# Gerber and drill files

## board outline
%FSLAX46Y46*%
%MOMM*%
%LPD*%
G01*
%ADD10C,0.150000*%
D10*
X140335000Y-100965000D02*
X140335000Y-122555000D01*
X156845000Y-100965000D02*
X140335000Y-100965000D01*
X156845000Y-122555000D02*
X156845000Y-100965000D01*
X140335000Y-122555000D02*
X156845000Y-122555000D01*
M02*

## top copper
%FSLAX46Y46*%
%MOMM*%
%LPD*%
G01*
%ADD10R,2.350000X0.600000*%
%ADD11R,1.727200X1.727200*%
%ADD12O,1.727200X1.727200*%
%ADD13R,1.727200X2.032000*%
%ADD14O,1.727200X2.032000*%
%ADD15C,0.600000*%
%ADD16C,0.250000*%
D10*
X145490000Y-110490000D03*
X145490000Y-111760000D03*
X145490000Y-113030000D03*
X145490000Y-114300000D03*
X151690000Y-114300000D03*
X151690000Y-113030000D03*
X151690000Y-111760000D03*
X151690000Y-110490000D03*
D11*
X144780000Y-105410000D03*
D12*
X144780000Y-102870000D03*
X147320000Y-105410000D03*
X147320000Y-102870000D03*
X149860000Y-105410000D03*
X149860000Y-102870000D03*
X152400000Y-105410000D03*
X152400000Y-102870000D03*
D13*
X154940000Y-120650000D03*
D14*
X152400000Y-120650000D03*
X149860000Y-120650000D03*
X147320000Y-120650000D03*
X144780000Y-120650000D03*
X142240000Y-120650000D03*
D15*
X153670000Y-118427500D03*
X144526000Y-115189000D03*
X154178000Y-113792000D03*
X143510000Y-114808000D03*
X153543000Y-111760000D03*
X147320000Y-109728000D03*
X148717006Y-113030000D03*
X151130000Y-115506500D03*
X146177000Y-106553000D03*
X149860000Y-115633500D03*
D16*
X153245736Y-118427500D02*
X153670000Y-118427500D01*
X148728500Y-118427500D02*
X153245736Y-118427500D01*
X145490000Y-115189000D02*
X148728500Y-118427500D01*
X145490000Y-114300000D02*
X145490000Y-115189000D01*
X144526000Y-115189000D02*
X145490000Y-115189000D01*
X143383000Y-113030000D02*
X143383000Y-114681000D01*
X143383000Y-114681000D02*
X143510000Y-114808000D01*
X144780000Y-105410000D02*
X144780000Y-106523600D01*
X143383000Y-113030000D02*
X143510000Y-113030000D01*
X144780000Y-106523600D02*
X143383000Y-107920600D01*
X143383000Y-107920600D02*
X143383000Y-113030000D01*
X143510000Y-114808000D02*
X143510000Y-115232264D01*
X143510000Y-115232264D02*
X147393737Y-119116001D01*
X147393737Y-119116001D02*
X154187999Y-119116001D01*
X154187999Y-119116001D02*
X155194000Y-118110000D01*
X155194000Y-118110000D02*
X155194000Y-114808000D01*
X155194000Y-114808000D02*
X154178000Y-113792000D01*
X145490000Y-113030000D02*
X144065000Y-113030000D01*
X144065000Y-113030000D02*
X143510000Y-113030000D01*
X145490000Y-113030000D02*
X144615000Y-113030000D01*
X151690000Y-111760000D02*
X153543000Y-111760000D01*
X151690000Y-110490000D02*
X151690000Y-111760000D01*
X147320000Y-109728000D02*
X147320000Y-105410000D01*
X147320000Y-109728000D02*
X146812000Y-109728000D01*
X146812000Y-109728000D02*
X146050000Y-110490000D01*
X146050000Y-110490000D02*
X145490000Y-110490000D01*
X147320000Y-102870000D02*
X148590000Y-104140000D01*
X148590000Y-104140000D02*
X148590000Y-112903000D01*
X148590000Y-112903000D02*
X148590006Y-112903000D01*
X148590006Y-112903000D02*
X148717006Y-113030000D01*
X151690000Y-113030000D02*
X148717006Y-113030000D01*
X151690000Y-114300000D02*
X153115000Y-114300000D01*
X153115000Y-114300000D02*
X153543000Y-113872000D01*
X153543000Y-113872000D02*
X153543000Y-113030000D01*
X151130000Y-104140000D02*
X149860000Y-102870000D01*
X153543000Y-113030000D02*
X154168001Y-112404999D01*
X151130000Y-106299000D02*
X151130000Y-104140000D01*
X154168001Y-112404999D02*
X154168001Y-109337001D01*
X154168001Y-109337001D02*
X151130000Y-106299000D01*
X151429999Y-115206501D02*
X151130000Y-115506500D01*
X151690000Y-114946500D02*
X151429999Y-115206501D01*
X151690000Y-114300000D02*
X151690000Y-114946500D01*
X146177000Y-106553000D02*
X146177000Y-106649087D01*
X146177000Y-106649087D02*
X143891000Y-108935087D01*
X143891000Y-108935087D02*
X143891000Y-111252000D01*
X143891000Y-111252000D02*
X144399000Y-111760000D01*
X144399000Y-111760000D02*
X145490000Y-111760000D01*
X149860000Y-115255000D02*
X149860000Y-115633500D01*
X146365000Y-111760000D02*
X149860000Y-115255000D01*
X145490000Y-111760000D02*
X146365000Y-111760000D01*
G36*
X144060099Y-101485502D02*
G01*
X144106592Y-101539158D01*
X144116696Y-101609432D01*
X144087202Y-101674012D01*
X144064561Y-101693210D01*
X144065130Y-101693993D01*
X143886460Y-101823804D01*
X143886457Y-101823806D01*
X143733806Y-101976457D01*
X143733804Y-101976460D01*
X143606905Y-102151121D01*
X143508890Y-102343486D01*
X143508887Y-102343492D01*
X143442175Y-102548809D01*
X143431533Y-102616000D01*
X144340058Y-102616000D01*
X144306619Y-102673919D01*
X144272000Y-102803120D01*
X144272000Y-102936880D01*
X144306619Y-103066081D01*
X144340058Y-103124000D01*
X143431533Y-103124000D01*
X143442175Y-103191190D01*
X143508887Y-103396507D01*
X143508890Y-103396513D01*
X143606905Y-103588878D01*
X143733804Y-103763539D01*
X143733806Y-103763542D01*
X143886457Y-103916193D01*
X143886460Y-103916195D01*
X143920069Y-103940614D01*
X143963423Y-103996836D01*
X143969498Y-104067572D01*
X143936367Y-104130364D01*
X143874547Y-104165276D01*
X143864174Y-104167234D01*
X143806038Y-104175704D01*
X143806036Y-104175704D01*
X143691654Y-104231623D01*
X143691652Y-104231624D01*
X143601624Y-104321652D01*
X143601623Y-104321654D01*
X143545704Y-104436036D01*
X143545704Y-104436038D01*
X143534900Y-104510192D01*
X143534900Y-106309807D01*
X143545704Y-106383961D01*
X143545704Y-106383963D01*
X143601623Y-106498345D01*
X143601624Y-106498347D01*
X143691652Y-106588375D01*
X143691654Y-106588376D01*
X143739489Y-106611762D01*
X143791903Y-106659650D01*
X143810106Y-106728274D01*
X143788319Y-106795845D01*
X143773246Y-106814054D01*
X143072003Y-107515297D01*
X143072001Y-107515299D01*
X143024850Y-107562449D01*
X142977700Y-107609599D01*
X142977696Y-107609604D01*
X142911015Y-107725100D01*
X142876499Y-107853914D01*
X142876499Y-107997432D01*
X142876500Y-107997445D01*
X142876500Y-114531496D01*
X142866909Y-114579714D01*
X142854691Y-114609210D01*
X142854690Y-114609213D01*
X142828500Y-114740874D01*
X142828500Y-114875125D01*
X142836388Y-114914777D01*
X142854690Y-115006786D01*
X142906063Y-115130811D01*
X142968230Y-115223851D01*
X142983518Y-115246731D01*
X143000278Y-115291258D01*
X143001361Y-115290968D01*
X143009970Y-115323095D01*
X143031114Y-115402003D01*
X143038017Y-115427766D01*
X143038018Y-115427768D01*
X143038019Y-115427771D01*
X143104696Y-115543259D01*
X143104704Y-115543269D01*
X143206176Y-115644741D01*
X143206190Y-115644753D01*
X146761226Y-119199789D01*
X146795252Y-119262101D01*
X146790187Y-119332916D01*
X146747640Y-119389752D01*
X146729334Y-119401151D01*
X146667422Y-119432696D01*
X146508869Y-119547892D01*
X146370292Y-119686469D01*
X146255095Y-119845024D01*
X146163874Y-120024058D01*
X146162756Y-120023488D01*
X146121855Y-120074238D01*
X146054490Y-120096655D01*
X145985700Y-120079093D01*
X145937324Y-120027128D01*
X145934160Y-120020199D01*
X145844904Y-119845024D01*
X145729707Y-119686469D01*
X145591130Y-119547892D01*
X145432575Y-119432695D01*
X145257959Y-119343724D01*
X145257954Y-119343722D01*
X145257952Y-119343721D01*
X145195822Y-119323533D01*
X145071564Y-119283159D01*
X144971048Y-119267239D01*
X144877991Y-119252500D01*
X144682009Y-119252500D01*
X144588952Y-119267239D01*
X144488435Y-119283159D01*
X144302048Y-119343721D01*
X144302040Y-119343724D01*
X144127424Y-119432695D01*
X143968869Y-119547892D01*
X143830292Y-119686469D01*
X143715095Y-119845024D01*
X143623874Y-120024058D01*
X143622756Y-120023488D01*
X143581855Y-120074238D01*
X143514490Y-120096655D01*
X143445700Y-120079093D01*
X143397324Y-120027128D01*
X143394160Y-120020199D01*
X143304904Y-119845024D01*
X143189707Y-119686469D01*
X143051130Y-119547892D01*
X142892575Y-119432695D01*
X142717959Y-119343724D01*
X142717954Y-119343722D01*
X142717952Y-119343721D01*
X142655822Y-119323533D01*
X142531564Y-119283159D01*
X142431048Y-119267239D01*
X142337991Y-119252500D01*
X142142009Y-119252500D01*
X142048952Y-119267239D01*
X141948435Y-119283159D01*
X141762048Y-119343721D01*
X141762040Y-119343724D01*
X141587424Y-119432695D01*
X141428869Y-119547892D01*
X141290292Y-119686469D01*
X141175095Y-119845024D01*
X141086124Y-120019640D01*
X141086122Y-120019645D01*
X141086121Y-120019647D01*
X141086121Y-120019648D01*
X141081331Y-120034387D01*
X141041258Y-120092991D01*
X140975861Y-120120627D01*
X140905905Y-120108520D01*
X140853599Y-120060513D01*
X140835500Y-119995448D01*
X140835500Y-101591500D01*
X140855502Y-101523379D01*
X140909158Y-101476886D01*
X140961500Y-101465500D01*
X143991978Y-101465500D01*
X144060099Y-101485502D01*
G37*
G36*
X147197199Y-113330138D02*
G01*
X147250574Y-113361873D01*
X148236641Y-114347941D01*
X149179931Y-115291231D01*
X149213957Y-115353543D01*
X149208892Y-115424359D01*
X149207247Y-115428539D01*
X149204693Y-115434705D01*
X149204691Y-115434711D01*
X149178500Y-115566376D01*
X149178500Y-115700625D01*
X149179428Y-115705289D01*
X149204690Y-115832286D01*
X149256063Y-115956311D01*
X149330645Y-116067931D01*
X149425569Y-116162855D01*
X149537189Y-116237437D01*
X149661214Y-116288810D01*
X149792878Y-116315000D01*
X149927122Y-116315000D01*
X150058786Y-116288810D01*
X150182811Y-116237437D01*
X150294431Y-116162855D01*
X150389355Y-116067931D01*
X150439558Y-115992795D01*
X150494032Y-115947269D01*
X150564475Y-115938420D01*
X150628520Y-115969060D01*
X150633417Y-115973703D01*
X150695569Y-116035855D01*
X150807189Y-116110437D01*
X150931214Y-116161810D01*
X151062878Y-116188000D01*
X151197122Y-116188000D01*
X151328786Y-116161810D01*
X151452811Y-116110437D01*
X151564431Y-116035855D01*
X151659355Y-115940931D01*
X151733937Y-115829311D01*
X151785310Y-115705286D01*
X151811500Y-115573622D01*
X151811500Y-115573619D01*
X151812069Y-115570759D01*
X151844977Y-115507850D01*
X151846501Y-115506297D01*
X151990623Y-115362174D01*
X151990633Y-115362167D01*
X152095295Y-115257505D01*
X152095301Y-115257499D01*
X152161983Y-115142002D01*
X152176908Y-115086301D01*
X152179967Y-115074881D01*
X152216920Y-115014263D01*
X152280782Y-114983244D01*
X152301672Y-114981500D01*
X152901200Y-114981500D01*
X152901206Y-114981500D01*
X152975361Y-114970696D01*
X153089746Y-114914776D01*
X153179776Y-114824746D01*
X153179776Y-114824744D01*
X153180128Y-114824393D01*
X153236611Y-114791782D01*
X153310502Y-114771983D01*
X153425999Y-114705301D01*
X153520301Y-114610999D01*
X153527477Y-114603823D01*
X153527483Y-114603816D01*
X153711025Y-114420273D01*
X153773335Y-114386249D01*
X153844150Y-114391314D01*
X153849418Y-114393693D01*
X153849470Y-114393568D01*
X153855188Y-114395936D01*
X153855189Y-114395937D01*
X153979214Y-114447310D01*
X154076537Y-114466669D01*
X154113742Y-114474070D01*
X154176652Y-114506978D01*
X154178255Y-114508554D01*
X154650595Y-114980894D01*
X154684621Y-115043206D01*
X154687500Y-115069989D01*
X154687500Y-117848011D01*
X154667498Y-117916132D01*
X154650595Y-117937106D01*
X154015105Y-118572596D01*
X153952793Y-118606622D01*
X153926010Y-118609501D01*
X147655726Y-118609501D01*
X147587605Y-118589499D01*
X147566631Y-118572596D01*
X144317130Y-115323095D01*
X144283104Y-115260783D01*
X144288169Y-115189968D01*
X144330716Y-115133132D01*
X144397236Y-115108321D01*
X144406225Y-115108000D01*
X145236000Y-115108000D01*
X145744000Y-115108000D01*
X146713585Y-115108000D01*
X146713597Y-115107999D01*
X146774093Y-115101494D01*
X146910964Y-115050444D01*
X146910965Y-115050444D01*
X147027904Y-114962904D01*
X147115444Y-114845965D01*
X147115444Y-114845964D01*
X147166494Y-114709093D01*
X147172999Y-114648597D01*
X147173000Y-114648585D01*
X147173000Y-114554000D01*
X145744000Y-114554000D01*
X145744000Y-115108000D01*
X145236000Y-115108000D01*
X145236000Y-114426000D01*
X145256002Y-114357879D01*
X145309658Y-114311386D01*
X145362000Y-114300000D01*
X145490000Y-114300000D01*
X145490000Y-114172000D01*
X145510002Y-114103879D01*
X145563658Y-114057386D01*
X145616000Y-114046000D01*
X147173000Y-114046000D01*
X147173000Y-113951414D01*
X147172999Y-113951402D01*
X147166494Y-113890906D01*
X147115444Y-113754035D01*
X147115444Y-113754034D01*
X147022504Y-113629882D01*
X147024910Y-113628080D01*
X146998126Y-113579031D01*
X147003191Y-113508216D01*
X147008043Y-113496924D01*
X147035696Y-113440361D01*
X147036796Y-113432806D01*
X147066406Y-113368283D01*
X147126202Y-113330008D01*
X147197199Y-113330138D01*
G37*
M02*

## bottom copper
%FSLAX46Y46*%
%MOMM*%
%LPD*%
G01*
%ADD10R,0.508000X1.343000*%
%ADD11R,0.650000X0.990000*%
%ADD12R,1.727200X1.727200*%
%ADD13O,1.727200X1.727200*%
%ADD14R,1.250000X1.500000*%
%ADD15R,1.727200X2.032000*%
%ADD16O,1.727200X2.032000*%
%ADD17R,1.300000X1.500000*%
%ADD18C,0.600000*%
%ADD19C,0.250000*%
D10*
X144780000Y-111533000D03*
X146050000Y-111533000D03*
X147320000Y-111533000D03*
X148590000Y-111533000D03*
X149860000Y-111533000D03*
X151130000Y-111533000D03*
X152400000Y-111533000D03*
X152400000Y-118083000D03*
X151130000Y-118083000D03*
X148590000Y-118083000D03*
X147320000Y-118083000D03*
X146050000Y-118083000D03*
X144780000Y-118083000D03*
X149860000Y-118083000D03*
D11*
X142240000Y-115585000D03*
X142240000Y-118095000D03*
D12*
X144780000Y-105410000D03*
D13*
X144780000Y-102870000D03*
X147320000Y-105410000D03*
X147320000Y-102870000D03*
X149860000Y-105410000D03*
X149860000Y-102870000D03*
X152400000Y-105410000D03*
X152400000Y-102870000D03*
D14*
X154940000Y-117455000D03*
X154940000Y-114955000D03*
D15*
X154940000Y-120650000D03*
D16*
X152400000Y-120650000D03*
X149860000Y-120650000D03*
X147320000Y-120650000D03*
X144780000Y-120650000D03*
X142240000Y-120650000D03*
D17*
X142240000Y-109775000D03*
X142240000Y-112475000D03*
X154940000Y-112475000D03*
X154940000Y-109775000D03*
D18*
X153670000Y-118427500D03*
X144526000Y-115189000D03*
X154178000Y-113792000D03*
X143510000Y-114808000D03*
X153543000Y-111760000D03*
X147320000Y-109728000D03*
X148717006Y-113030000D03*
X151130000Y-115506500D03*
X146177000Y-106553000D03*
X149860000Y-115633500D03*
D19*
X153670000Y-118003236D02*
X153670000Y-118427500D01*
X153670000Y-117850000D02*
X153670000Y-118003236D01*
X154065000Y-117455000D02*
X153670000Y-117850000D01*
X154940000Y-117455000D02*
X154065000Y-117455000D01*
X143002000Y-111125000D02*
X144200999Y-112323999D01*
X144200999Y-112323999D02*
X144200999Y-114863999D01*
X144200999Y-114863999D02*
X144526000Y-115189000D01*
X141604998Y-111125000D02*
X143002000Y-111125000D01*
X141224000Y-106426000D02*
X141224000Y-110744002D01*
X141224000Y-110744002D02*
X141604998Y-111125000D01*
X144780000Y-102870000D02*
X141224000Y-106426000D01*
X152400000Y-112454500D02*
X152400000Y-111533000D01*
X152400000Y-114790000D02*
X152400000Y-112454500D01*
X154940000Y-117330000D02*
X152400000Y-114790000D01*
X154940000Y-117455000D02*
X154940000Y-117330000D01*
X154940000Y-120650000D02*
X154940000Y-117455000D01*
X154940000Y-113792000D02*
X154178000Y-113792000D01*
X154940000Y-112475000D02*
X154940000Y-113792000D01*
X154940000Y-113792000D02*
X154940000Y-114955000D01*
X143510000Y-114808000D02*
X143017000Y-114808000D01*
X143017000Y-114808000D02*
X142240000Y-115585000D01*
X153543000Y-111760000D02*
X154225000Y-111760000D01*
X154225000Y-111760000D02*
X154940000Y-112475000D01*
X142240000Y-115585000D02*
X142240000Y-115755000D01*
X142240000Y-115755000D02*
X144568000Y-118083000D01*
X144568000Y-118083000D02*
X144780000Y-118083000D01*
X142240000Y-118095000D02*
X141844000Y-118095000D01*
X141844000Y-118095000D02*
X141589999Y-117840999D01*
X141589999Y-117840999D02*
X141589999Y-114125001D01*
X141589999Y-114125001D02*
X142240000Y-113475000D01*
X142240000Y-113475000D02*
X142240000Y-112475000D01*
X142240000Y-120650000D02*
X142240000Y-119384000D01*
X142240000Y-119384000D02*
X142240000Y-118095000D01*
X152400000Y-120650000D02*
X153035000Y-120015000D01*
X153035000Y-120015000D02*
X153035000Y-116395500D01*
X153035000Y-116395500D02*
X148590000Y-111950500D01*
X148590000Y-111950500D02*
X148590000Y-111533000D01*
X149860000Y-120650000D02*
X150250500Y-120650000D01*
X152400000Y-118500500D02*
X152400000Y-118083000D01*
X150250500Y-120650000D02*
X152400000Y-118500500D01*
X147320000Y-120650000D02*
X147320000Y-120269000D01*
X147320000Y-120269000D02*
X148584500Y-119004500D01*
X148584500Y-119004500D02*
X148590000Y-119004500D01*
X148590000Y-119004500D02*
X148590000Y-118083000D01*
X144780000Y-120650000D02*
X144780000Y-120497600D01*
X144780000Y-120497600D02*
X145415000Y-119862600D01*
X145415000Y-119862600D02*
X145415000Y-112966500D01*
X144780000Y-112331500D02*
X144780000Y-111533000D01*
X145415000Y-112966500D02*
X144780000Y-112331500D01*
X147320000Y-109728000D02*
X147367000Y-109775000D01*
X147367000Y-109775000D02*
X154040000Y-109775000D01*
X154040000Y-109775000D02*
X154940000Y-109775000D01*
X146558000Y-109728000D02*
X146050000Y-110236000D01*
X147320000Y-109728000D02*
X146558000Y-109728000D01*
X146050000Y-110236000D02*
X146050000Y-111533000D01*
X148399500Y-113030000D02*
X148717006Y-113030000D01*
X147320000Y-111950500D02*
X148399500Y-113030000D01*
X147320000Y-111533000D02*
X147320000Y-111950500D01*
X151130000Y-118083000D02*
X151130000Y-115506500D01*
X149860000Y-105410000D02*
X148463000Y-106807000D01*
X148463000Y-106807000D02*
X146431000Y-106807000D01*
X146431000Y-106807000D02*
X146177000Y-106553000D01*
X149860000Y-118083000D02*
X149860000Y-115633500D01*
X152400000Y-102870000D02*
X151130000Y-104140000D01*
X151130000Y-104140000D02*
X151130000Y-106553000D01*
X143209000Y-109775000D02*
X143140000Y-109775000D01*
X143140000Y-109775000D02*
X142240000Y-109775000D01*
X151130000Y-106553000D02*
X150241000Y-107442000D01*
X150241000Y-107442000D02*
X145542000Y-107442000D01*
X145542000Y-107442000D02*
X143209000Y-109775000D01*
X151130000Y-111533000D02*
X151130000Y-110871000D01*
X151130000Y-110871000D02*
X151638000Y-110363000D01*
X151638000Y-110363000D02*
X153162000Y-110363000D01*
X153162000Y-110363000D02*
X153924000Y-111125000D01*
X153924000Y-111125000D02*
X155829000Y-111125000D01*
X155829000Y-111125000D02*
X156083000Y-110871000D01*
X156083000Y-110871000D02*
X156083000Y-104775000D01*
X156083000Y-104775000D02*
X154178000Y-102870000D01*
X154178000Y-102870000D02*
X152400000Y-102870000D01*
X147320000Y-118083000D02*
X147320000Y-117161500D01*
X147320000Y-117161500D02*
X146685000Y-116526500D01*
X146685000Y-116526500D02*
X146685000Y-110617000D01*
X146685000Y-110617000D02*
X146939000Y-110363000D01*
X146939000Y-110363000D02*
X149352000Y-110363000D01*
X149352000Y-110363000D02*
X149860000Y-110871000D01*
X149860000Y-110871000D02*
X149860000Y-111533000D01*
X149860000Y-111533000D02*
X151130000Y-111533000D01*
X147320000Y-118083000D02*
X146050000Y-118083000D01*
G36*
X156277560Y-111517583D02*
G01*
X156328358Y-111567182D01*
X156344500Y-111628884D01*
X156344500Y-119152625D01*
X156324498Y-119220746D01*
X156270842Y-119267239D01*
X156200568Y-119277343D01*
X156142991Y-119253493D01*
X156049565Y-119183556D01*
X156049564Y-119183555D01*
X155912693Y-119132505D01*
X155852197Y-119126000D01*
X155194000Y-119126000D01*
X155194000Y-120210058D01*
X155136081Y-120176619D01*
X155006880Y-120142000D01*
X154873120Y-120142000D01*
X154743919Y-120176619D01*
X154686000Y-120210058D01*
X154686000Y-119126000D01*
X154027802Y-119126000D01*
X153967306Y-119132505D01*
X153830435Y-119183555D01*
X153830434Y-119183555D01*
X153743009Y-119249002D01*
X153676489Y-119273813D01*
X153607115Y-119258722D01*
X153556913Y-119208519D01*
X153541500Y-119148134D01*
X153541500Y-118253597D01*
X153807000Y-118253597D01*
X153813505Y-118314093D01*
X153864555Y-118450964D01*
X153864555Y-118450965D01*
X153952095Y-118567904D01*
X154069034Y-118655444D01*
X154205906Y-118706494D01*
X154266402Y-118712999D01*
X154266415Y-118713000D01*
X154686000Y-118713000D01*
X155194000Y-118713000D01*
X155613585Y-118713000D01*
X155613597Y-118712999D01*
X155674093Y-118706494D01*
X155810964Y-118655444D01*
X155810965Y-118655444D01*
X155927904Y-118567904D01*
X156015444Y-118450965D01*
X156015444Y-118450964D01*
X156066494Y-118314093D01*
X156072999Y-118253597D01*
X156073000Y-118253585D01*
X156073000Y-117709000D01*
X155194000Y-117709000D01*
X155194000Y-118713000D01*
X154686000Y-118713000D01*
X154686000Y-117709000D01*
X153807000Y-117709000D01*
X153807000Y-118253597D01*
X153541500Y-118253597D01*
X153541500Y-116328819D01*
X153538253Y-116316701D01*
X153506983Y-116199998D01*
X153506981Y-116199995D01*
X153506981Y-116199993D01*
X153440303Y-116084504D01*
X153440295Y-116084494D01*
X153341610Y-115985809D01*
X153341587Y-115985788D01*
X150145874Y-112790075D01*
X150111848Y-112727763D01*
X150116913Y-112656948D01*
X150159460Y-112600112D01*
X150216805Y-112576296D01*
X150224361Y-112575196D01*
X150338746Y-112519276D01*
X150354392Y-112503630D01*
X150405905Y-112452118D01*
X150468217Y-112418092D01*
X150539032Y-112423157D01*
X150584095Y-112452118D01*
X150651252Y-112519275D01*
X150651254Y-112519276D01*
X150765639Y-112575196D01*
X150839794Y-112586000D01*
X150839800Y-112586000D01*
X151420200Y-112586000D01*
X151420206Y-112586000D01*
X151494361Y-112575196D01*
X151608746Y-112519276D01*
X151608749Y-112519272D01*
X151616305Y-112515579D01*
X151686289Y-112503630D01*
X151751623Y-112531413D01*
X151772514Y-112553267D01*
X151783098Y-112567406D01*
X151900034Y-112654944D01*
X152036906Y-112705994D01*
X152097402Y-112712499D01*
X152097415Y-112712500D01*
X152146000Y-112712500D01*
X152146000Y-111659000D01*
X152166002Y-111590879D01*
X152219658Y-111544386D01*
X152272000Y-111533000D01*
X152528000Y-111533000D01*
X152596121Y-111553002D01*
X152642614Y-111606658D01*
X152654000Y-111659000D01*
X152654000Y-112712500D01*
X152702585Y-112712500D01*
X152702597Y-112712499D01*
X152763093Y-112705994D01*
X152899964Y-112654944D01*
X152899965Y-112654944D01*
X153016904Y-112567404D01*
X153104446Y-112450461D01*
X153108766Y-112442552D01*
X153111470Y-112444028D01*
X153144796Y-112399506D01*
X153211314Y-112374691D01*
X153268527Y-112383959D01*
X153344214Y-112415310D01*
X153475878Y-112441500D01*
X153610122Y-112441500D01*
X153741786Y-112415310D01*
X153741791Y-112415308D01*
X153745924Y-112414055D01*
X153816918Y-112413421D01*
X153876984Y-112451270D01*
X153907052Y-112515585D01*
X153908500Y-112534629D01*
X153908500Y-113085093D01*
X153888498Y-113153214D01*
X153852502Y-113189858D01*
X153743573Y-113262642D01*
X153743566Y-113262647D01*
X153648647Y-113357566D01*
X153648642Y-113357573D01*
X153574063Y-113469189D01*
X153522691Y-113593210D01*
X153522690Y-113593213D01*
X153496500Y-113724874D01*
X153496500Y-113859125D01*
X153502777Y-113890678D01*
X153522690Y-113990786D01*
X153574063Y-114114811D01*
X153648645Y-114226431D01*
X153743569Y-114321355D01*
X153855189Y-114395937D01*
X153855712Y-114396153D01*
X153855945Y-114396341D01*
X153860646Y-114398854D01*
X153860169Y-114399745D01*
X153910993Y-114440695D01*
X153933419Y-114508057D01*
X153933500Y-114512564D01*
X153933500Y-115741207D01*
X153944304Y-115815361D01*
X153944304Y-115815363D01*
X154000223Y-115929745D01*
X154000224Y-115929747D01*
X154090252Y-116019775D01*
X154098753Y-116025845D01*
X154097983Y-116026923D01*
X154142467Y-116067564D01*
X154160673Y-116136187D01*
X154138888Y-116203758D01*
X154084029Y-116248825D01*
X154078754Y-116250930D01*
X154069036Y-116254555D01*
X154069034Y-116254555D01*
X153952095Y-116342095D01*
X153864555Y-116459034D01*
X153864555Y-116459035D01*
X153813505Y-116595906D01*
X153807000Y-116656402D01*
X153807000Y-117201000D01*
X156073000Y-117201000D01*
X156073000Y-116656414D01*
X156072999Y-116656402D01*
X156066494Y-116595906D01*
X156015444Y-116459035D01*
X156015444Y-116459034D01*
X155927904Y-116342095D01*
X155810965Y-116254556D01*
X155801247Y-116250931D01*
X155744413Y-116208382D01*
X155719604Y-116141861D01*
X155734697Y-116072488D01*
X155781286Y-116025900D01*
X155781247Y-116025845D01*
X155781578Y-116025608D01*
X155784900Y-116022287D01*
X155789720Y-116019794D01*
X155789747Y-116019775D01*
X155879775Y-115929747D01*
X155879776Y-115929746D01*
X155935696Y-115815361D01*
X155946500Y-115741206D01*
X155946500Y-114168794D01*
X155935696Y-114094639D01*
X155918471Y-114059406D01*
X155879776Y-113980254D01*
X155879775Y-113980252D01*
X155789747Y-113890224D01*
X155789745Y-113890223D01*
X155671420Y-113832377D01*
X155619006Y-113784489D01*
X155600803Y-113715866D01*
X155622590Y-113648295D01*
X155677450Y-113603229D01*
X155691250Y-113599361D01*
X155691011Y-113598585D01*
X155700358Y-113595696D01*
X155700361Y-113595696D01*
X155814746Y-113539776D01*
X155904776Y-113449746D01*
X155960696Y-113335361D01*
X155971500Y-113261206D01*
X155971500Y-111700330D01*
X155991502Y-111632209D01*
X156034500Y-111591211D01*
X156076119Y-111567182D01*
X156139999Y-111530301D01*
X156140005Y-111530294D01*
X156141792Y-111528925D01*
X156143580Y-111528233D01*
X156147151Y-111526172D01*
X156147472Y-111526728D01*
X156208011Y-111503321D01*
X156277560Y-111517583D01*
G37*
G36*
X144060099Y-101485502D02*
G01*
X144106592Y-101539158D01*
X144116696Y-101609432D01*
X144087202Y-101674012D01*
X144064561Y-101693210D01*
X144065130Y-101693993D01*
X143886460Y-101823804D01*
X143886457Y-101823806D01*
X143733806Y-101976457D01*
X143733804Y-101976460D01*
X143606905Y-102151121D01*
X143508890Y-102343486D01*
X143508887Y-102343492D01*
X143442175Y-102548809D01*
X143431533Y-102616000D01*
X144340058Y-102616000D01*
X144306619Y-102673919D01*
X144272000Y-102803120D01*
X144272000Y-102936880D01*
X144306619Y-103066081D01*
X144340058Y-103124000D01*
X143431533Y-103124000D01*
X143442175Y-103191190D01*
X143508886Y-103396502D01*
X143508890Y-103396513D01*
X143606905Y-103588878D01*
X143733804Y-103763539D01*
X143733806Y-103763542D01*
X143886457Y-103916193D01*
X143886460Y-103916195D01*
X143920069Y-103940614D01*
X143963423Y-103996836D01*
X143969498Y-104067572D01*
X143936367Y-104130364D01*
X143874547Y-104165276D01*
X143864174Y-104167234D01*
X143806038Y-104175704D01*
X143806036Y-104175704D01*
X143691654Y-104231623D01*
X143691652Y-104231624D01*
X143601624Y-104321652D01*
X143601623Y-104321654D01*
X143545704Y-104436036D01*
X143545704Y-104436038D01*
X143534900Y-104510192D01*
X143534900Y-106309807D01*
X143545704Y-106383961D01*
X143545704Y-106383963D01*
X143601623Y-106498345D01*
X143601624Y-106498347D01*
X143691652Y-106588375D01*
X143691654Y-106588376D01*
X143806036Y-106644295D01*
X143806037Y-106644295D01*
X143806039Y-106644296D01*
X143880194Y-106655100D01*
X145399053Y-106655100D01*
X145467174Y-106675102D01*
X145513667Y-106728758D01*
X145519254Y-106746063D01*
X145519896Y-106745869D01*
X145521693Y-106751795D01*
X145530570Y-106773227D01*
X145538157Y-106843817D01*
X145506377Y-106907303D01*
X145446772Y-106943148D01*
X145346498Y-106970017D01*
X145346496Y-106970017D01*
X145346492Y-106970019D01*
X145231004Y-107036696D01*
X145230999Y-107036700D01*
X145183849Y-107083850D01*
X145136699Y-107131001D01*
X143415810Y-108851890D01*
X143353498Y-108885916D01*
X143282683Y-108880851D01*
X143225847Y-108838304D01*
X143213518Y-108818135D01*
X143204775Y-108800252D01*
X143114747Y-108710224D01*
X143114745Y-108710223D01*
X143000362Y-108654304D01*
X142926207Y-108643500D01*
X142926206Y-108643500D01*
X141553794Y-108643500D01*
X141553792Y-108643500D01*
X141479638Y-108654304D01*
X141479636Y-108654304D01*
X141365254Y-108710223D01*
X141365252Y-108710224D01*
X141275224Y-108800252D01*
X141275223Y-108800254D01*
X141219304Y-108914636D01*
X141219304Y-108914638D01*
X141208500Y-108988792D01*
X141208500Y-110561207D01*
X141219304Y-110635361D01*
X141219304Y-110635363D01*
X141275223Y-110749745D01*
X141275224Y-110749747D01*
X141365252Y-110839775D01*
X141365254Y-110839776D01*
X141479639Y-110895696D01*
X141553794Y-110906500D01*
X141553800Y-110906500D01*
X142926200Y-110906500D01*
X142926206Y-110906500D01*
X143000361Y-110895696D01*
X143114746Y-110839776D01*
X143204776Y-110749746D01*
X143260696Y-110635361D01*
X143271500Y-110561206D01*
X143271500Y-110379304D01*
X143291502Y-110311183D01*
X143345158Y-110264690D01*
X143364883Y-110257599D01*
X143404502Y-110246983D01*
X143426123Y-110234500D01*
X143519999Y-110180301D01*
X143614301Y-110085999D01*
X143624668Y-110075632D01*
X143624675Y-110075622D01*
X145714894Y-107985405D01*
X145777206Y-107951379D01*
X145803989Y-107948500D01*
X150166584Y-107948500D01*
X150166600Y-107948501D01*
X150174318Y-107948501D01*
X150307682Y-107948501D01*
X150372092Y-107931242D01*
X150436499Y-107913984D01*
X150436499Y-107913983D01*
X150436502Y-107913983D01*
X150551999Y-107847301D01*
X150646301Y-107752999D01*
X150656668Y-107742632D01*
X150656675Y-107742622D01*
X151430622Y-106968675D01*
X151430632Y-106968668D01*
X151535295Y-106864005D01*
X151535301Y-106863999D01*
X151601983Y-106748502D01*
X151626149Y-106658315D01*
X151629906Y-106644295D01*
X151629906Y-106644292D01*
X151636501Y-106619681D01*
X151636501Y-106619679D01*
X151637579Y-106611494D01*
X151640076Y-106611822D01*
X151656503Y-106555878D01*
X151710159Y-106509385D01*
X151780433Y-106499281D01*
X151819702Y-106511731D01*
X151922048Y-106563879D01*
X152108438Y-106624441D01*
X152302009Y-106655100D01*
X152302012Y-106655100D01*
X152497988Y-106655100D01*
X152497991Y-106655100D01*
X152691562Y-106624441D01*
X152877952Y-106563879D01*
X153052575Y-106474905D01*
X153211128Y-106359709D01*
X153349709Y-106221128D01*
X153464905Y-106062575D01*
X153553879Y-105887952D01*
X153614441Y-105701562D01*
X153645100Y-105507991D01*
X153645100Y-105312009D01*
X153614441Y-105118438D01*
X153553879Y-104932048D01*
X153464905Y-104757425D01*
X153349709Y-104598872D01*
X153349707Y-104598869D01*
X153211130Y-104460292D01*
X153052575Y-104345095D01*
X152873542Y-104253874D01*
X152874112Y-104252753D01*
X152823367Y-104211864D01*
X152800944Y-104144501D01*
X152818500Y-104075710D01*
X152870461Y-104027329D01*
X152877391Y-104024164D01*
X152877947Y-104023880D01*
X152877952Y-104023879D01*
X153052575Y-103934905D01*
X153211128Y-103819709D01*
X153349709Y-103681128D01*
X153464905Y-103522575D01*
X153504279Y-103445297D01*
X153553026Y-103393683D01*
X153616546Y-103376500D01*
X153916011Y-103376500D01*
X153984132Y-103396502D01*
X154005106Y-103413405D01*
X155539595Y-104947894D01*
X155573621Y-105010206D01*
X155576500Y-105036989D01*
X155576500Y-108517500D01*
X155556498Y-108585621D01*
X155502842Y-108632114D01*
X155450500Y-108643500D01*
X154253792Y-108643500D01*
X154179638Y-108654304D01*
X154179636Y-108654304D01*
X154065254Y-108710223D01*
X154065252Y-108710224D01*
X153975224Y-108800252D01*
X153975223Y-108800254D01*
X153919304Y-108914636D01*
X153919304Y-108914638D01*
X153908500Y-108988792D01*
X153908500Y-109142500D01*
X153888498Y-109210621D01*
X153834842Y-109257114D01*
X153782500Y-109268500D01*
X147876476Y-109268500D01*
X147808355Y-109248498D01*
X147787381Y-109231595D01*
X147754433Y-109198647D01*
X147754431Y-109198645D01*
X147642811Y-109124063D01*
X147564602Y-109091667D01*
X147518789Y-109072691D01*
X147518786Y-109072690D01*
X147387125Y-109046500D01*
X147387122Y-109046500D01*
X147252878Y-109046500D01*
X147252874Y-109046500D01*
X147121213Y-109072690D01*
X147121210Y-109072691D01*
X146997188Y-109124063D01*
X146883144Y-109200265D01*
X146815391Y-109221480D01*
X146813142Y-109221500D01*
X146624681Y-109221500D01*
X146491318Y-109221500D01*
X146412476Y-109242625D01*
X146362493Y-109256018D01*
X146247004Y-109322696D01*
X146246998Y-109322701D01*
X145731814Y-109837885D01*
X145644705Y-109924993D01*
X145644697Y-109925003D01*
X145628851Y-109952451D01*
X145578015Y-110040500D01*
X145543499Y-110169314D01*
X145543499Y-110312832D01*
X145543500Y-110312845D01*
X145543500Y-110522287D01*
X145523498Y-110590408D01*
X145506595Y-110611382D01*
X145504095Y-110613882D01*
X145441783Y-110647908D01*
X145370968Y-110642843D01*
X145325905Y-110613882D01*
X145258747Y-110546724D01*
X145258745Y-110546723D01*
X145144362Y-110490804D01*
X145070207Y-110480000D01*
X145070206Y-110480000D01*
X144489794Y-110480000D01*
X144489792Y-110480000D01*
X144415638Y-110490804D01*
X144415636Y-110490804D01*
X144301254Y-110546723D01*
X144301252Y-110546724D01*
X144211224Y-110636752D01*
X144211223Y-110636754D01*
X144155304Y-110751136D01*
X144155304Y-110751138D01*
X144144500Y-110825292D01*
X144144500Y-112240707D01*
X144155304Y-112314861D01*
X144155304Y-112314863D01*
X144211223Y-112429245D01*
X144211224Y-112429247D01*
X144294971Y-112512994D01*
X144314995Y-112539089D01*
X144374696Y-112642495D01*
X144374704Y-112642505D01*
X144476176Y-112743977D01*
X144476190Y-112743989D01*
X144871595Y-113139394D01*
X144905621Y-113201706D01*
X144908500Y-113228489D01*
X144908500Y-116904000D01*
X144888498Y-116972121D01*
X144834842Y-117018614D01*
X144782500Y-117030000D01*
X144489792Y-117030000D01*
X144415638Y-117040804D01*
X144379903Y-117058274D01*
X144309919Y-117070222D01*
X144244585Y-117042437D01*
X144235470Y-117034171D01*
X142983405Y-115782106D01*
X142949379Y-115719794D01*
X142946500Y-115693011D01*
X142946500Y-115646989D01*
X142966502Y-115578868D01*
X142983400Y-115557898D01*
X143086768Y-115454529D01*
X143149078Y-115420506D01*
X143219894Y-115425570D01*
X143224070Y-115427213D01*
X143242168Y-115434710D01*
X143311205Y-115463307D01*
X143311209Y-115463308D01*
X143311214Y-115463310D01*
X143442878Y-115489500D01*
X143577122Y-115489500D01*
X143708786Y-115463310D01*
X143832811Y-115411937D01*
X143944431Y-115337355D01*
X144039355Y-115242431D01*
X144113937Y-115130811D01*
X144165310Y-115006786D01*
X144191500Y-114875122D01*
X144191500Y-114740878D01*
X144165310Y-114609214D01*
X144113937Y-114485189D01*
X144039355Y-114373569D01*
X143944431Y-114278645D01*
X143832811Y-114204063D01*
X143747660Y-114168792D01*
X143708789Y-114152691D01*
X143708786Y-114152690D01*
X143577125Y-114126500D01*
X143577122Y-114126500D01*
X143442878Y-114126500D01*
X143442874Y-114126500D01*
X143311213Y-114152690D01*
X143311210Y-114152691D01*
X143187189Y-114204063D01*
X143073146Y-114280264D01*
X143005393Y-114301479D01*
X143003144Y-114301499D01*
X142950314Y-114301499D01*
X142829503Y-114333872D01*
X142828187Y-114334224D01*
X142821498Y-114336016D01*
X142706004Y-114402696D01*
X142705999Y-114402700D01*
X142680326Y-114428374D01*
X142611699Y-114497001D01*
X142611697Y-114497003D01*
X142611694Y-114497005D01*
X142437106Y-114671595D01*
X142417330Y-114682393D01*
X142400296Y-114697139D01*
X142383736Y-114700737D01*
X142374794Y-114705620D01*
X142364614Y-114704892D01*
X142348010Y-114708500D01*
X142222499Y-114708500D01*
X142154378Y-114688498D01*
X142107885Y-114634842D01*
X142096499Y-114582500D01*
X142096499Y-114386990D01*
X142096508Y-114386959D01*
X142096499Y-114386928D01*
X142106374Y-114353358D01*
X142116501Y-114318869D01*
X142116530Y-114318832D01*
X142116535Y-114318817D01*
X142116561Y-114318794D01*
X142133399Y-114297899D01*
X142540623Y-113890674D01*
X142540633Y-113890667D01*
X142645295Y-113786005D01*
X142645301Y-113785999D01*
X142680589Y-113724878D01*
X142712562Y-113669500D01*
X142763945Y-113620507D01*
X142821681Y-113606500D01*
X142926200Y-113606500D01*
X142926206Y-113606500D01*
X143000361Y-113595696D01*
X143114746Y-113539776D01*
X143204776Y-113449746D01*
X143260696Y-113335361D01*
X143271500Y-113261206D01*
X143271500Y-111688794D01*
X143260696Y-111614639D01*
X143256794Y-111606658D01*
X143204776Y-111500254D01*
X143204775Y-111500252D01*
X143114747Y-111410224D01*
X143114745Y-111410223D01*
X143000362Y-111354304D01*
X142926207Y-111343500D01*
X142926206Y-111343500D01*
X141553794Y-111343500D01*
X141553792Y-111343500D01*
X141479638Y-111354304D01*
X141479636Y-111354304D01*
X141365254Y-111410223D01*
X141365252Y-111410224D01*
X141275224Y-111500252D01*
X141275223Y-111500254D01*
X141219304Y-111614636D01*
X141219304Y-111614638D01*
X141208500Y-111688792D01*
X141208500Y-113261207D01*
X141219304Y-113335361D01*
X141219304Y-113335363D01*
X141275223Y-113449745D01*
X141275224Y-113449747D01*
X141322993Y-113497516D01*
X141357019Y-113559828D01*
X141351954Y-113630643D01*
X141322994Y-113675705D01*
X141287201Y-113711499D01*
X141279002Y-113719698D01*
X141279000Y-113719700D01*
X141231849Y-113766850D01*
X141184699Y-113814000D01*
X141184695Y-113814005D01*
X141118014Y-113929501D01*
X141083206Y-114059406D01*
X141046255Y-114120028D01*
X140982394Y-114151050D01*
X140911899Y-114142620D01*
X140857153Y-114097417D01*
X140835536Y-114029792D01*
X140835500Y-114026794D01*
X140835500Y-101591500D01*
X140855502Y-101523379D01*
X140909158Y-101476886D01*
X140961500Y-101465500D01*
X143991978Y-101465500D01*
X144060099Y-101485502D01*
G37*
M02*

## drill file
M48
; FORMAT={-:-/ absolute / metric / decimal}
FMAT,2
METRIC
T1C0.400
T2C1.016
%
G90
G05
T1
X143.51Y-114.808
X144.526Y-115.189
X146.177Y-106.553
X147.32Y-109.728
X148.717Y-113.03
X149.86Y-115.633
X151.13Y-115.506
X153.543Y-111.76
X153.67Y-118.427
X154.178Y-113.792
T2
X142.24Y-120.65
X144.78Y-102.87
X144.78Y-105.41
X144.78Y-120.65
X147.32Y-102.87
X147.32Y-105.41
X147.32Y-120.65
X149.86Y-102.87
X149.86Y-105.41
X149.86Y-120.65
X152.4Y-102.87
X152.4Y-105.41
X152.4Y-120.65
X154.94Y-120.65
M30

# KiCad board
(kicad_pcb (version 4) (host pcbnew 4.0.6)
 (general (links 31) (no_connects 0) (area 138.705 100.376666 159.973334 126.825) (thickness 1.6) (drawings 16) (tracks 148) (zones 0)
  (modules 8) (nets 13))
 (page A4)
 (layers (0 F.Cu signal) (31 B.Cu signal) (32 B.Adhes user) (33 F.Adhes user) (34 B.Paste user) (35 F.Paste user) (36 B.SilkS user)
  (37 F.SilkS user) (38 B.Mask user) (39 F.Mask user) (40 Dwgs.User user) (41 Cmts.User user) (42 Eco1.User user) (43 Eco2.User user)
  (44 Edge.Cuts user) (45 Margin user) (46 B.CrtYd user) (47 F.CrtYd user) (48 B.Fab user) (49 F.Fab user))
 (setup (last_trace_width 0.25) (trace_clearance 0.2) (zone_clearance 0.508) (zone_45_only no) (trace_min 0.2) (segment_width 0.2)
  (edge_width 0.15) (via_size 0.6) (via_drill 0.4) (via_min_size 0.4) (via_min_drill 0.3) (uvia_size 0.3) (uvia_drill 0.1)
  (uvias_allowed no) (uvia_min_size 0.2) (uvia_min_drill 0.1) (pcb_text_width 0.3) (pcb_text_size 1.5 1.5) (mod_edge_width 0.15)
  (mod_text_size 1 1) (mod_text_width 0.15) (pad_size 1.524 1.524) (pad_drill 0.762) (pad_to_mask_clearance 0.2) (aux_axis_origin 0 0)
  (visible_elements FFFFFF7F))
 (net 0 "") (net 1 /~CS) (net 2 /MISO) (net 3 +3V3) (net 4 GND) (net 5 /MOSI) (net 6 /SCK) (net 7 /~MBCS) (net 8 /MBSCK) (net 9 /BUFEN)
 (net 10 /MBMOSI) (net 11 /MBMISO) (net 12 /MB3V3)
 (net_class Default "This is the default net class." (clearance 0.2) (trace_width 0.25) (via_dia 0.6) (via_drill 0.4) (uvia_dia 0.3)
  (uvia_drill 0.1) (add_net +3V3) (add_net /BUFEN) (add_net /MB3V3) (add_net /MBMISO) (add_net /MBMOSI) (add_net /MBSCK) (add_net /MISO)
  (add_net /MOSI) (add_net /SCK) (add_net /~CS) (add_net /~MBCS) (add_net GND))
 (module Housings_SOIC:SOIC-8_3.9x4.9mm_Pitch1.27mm (layer F.Cu) (at 148.59 112.395)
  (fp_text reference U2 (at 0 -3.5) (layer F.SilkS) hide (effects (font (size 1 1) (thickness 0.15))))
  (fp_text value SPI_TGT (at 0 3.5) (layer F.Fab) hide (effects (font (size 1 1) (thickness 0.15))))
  (pad 1 smd rect (at -3.1 -1.905) (size 2.35 0.6) (layers F.Cu F.Paste F.Mask) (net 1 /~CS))
  (pad 2 smd rect (at -3.1 -0.635) (size 2.35 0.6) (layers F.Cu F.Paste F.Mask) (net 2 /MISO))
  (pad 3 smd rect (at -3.1 0.635) (size 2.35 0.6) (layers F.Cu F.Paste F.Mask) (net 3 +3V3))
  (pad 4 smd rect (at -3.1 1.905) (size 2.35 0.6) (layers F.Cu F.Paste F.Mask) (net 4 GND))
  (pad 5 smd rect (at 3.1 1.905) (size 2.35 0.6) (layers F.Cu F.Paste F.Mask) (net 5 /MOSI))
  (pad 6 smd rect (at 3.1 0.635) (size 2.35 0.6) (layers F.Cu F.Paste F.Mask) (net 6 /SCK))
  (pad 7 smd rect (at 3.1 -0.635) (size 2.35 0.6) (layers F.Cu F.Paste F.Mask) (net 3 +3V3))
  (pad 8 smd rect (at 3.1 -1.905) (size 2.35 0.6) (layers F.Cu F.Paste F.Mask) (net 3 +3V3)))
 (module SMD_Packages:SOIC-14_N (layer B.Cu) (at 148.59 114.935)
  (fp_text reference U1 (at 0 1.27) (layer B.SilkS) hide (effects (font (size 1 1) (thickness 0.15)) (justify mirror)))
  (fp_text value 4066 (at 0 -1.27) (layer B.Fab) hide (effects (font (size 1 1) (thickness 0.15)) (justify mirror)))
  (pad 1 smd rect (at -3.81 -3.402) (size 0.508 1.343) (layers B.Cu B.Paste B.Mask) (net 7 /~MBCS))
  (pad 2 smd rect (at -2.54 -3.402) (size 0.508 1.343) (layers B.Cu B.Paste B.Mask) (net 1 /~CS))
  (pad 3 smd rect (at -1.27 -3.402) (size 0.508 1.343) (layers B.Cu B.Paste B.Mask) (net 6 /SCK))
  (pad 4 smd rect (at 0 -3.402) (size 0.508 1.343) (layers B.Cu B.Paste B.Mask) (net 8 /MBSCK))
  (pad 5 smd rect (at 1.27 -3.402) (size 0.508 1.343) (layers B.Cu B.Paste B.Mask) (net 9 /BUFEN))
  (pad 6 smd rect (at 2.54 -3.402) (size 0.508 1.343) (layers B.Cu B.Paste B.Mask) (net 9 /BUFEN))
  (pad 7 smd rect (at 3.81 -3.402) (size 0.508 1.343) (layers B.Cu B.Paste B.Mask) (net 4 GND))
  (pad 8 smd rect (at 3.81 3.148) (size 0.508 1.343) (layers B.Cu B.Paste B.Mask) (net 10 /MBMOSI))
  (pad 9 smd rect (at 2.54 3.148) (size 0.508 1.343) (layers B.Cu B.Paste B.Mask) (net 5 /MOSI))
  (pad 11 smd rect (at 0 3.148) (size 0.508 1.343) (layers B.Cu B.Paste B.Mask) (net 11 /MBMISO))
  (pad 12 smd rect (at -1.27 3.148) (size 0.508 1.343) (layers B.Cu B.Paste B.Mask) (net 9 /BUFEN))
  (pad 13 smd rect (at -2.54 3.148) (size 0.508 1.343) (layers B.Cu B.Paste B.Mask) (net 9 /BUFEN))
  (pad 14 smd rect (at -3.81 3.148) (size 0.508 1.343) (layers B.Cu B.Paste B.Mask) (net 3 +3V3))
  (pad 10 smd rect (at 1.27 3.148 180) (size 0.508 1.343) (layers B.Cu B.Paste B.Mask) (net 2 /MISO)))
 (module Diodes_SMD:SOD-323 (layer B.Cu) (at 142.24 116.84 270)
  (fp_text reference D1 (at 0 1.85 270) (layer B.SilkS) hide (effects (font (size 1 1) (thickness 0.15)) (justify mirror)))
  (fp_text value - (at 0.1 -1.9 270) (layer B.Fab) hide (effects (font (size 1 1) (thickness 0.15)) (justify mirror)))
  (pad 1 smd rect (at -1.255 0 270) (size 0.99 0.65) (layers B.Cu B.Paste B.Mask) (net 3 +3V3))
  (pad 2 smd rect (at 1.255 0 270) (size 0.99 0.65) (layers B.Cu B.Paste B.Mask) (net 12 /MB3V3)))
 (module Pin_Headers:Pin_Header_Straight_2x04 (layer F.Cu) (at 144.78 105.41 90)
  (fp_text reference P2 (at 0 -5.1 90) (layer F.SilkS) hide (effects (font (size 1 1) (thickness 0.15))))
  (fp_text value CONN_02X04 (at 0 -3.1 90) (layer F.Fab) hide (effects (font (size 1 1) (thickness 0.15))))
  (pad 1 thru_hole rect (at 0 0 90) (size 1.7272 1.7272) (drill 1.016) (layers *.Cu *.Mask F.SilkS) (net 3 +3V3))
  (pad 2 thru_hole oval (at 2.54 0 90) (size 1.7272 1.7272) (drill 1.016) (layers *.Cu *.Mask F.SilkS) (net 4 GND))
  (pad 3 thru_hole oval (at 0 2.54 90) (size 1.7272 1.7272) (drill 1.016) (layers *.Cu *.Mask F.SilkS) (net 1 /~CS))
  (pad 4 thru_hole oval (at 2.54 2.54 90) (size 1.7272 1.7272) (drill 1.016) (layers *.Cu *.Mask F.SilkS) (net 6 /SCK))
  (pad 5 thru_hole oval (at 0 5.08 90) (size 1.7272 1.7272) (drill 1.016) (layers *.Cu *.Mask F.SilkS) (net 2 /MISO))
  (pad 6 thru_hole oval (at 2.54 5.08 90) (size 1.7272 1.7272) (drill 1.016) (layers *.Cu *.Mask F.SilkS) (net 5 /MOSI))
  (pad 7 thru_hole oval (at 0 7.62 90) (size 1.7272 1.7272) (drill 1.016) (layers *.Cu *.Mask F.SilkS))
  (pad 8 thru_hole oval (at 2.54 7.62 90) (size 1.7272 1.7272) (drill 1.016) (layers *.Cu *.Mask F.SilkS) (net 9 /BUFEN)))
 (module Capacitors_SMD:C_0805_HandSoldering (layer B.Cu) (at 154.94 116.205 90)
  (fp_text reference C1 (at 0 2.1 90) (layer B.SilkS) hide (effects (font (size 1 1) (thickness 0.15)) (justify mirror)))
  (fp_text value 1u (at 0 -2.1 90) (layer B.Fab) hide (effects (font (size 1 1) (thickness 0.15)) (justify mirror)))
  (pad 1 smd rect (at -1.25 0 90) (size 1.5 1.25) (layers B.Cu B.Paste B.Mask) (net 4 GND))
  (pad 2 smd rect (at 1.25 0 90) (size 1.5 1.25) (layers B.Cu B.Paste B.Mask) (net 3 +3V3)))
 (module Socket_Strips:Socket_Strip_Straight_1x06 (layer F.Cu) (at 154.94 120.65 180)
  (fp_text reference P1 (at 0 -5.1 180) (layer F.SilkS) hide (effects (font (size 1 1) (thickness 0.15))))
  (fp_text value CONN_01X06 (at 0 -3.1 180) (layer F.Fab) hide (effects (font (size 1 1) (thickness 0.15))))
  (pad 1 thru_hole rect (at 0 0 180) (size 1.7272 2.032) (drill 1.016) (layers *.Cu *.Mask F.SilkS) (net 4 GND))
  (pad 2 thru_hole oval (at 2.54 0 180) (size 1.7272 2.032) (drill 1.016) (layers *.Cu *.Mask F.SilkS) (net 8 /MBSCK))
  (pad 3 thru_hole oval (at 5.08 0 180) (size 1.7272 2.032) (drill 1.016) (layers *.Cu *.Mask F.SilkS) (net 10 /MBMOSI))
  (pad 4 thru_hole oval (at 7.62 0 180) (size 1.7272 2.032) (drill 1.016) (layers *.Cu *.Mask F.SilkS) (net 11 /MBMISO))
  (pad 5 thru_hole oval (at 10.16 0 180) (size 1.7272 2.032) (drill 1.016) (layers *.Cu *.Mask F.SilkS) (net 7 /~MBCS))
  (pad 6 thru_hole oval (at 12.7 0 180) (size 1.7272 2.032) (drill 1.016) (layers *.Cu *.Mask F.SilkS) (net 12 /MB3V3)))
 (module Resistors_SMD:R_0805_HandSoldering (layer B.Cu) (at 142.24 111.125 270)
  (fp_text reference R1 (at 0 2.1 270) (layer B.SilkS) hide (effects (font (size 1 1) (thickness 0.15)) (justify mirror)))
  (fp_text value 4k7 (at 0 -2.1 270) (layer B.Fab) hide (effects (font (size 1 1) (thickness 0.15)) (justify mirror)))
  (pad 1 smd rect (at -1.35 0 270) (size 1.5 1.3) (layers B.Cu B.Paste B.Mask) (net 9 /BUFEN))
  (pad 2 smd rect (at 1.35 0 270) (size 1.5 1.3) (layers B.Cu B.Paste B.Mask) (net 12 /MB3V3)))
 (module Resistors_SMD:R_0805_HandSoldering (layer B.Cu) (at 154.94 111.125 90)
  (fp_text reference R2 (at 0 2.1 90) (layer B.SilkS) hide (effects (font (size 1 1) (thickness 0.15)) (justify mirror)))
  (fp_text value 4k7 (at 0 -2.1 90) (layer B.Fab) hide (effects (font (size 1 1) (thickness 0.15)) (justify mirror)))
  (pad 1 smd rect (at -1.35 0 90) (size 1.5 1.3) (layers B.Cu B.Paste B.Mask) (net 3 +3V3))
  (pad 2 smd rect (at 1.35 0 90) (size 1.5 1.3) (layers B.Cu B.Paste B.Mask) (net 1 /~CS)))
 (gr_line (start 140.335 100.965) (end 140.335 122.555) (layer Edge.Cuts) (width 0.15))
 (gr_line (start 156.845 100.965) (end 140.335 100.965) (layer Edge.Cuts) (width 0.15))
 (gr_line (start 156.845 122.555) (end 156.845 100.965) (layer Edge.Cuts) (width 0.15))
 (gr_line (start 140.335 122.555) (end 156.845 122.555) (angle 90) (layer Edge.Cuts) (width 0.15))
 (segment (start 153.245736 118.4275) (end 153.67 118.4275) (width 0.25) (layer F.Cu) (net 4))
 (segment (start 153.67 118.003236) (end 153.67 118.4275) (width 0.25) (layer B.Cu) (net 4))
 (segment (start 153.67 117.85) (end 153.67 118.003236) (width 0.25) (layer B.Cu) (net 4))
 (segment (start 154.065 117.455) (end 153.67 117.85) (width 0.25) (layer B.Cu) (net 4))
 (via (at 153.67 118.4275) (size 0.6) (drill 0.4) (layers F.Cu B.Cu) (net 4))
 (segment (start 148.7285 118.4275) (end 153.245736 118.4275) (width 0.25) (layer F.Cu) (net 4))
 (segment (start 145.49 115.189) (end 148.7285 118.4275) (width 0.25) (layer F.Cu) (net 4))
 (segment (start 154.94 117.455) (end 154.065 117.455) (width 0.25) (layer B.Cu) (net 4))
 (segment (start 145.49 114.3) (end 145.49 115.189) (width 0.25) (layer F.Cu) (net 4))
 (segment (start 144.526 115.189) (end 145.49 115.189) (width 0.25) (layer F.Cu) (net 4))
 (segment (start 143.002 111.125) (end 144.200999 112.323999) (width 0.25) (layer B.Cu) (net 4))
 (segment (start 144.200999 112.323999) (end 144.200999 114.863999) (width 0.25) (layer B.Cu) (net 4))
 (segment (start 144.200999 114.863999) (end 144.526 115.189) (width 0.25) (layer B.Cu) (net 4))
 (via (at 144.526 115.189) (size 0.6) (drill 0.4) (layers F.Cu B.Cu) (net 4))
 (segment (start 141.604998 111.125) (end 143.002 111.125) (width 0.25) (layer B.Cu) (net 4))
 (segment (start 141.224 106.426) (end 141.224 110.744002) (width 0.25) (layer B.Cu) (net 4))
 (segment (start 141.224 110.744002) (end 141.604998 111.125) (width 0.25) (layer B.Cu) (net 4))
 (segment (start 144.78 102.87) (end 141.224 106.426) (width 0.25) (layer B.Cu) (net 4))
 (segment (start 152.4 112.4545) (end 152.4 111.533) (width 0.25) (layer B.Cu) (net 4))
 (segment (start 152.4 114.79) (end 152.4 112.4545) (width 0.25) (layer B.Cu) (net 4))
 (segment (start 154.94 117.33) (end 152.4 114.79) (width 0.25) (layer B.Cu) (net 4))
 (segment (start 154.94 117.455) (end 154.94 117.33) (width 0.25) (layer B.Cu) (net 4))
 (segment (start 154.94 120.65) (end 154.94 117.455) (width 0.25) (layer B.Cu) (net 4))
 (segment (start 143.383 113.03) (end 143.383 114.681) (width 0.25) (layer F.Cu) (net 3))
 (segment (start 143.383 114.681) (end 143.51 114.808) (width 0.25) (layer F.Cu) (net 3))
 (segment (start 144.78 105.41) (end 144.78 106.5236) (width 0.25) (layer F.Cu) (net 3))
 (segment (start 143.383 113.03) (end 143.51 113.03) (width 0.25) (layer F.Cu) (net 3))
 (segment (start 144.78 106.5236) (end 143.383 107.9206) (width 0.25) (layer F.Cu) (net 3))
 (segment (start 143.383 107.9206) (end 143.383 113.03) (width 0.25) (layer F.Cu) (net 3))
 (segment (start 143.51 114.808) (end 143.51 115.232264) (width 0.25) (layer F.Cu) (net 3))
 (segment (start 143.51 115.232264) (end 147.393737 119.116001) (width 0.25) (layer F.Cu) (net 3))
 (segment (start 147.393737 119.116001) (end 154.187999 119.116001) (width 0.25) (layer F.Cu) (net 3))
 (segment (start 154.187999 119.116001) (end 155.194 118.11) (width 0.25) (layer F.Cu) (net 3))
 (segment (start 155.194 118.11) (end 155.194 114.808) (width 0.25) (layer F.Cu) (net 3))
 (segment (start 155.194 114.808) (end 154.178 113.792) (width 0.25) (layer F.Cu) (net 3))
 (via (at 154.178 113.792) (size 0.6) (drill 0.4) (layers F.Cu B.Cu) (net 3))
 (segment (start 154.94 113.792) (end 154.178 113.792) (width 0.25) (layer B.Cu) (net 3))
 (segment (start 154.94 112.475) (end 154.94 113.792) (width 0.25) (layer B.Cu) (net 3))
 (segment (start 154.94 113.792) (end 154.94 114.955) (width 0.25) (layer B.Cu) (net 3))
 (segment (start 145.49 113.03) (end 144.065 113.03) (width 0.25) (layer F.Cu) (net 3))
 (segment (start 144.065 113.03) (end 143.51 113.03) (width 0.25) (layer F.Cu) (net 3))
 (segment (start 143.51 114.808) (end 143.017 114.808) (width 0.25) (layer B.Cu) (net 3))
 (segment (start 143.017 114.808) (end 142.24 115.585) (width 0.25) (layer B.Cu) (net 3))
 (segment (start 145.49 113.03) (end 144.615 113.03) (width 0.25) (layer F.Cu) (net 3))
 (via (at 143.51 114.808) (size 0.6) (drill 0.4) (layers F.Cu B.Cu) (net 3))
 (segment (start 153.543 111.76) (end 154.225 111.76) (width 0.25) (layer B.Cu) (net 3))
 (segment (start 154.225 111.76) (end 154.94 112.475) (width 0.25) (layer B.Cu) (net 3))
 (segment (start 151.69 111.76) (end 153.543 111.76) (width 0.25) (layer F.Cu) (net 3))
 (via (at 153.543 111.76) (size 0.6) (drill 0.4) (layers F.Cu B.Cu) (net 3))
 (segment (start 151.69 110.49) (end 151.69 111.76) (width 0.25) (layer F.Cu) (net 3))
 (segment (start 142.24 115.585) (end 142.24 115.755) (width 0.25) (layer B.Cu) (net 3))
 (segment (start 142.24 115.755) (end 144.568 118.083) (width 0.25) (layer B.Cu) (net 3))
 (segment (start 144.568 118.083) (end 144.78 118.083) (width 0.25) (layer B.Cu) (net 3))
 (segment (start 142.24 118.095) (end 141.844 118.095) (width 0.25) (layer B.Cu) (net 12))
 (segment (start 141.844 118.095) (end 141.589999 117.840999) (width 0.25) (layer B.Cu) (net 12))
 (segment (start 141.589999 117.840999) (end 141.589999 114.125001) (width 0.25) (layer B.Cu) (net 12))
 (segment (start 141.589999 114.125001) (end 142.24 113.475) (width 0.25) (layer B.Cu) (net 12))
 (segment (start 142.24 113.475) (end 142.24 112.475) (width 0.25) (layer B.Cu) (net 12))
 (segment (start 142.24 120.65) (end 142.24 119.384) (width 0.25) (layer B.Cu) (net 12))
 (segment (start 142.24 119.384) (end 142.24 118.095) (width 0.25) (layer B.Cu) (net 12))
 (segment (start 152.4 120.65) (end 153.035 120.015) (width 0.25) (layer B.Cu) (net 8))
 (segment (start 153.035 120.015) (end 153.035 116.3955) (width 0.25) (layer B.Cu) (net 8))
 (segment (start 153.035 116.3955) (end 148.59 111.9505) (width 0.25) (layer B.Cu) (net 8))
 (segment (start 148.59 111.9505) (end 148.59 111.533) (width 0.25) (layer B.Cu) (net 8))
 (segment (start 149.86 120.65) (end 150.2505 120.65) (width 0.25) (layer B.Cu) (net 10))
 (segment (start 152.4 118.5005) (end 152.4 118.083) (width 0.25) (layer B.Cu) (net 10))
 (segment (start 150.2505 120.65) (end 152.4 118.5005) (width 0.25) (layer B.Cu) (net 10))
 (segment (start 147.32 120.65) (end 147.32 120.269) (width 0.25) (layer B.Cu) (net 11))
 (segment (start 147.32 120.269) (end 148.5845 119.0045) (width 0.25) (layer B.Cu) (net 11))
 (segment (start 148.5845 119.0045) (end 148.59 119.0045) (width 0.25) (layer B.Cu) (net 11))
 (segment (start 148.59 119.0045) (end 148.59 118.083) (width 0.25) (layer B.Cu) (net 11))
 (segment (start 144.78 120.65) (end 144.78 120.4976) (width 0.25) (layer B.Cu) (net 7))
 (segment (start 144.78 120.4976) (end 145.415 119.8626) (width 0.25) (layer B.Cu) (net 7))
 (segment (start 145.415 119.8626) (end 145.415 112.9665) (width 0.25) (layer B.Cu) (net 7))
 (segment (start 144.78 112.3315) (end 144.78 111.533) (width 0.25) (layer B.Cu) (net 7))
 (segment (start 145.415 112.9665) (end 144.78 112.3315) (width 0.25) (layer B.Cu) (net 7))
 (segment (start 147.32 109.728) (end 147.367 109.775) (width 0.25) (layer B.Cu) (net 1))
 (segment (start 147.367 109.775) (end 154.04 109.775) (width 0.25) (layer B.Cu) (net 1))
 (segment (start 154.04 109.775) (end 154.94 109.775) (width 0.25) (layer B.Cu) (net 1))
 (via (at 147.32 109.728) (size 0.6) (drill 0.4) (layers F.Cu B.Cu) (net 1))
 (segment (start 147.32 109.728) (end 147.32 105.41) (width 0.25) (layer F.Cu) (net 1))
 (segment (start 147.32 109.728) (end 146.812 109.728) (width 0.25) (layer F.Cu) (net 1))
 (segment (start 146.812 109.728) (end 146.05 110.49) (width 0.25) (layer F.Cu) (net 1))
 (segment (start 146.558 109.728) (end 146.05 110.236) (width 0.25) (layer B.Cu) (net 1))
 (segment (start 146.05 110.49) (end 145.49 110.49) (width 0.25) (layer F.Cu) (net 1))
 (segment (start 147.32 109.728) (end 146.558 109.728) (width 0.25) (layer B.Cu) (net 1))
 (segment (start 146.05 110.236) (end 146.05 111.533) (width 0.25) (layer B.Cu) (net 1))
 (segment (start 147.32 102.87) (end 148.59 104.14) (width 0.25) (layer F.Cu) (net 6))
 (segment (start 148.59 104.14) (end 148.59 112.903) (width 0.25) (layer F.Cu) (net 6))
 (segment (start 148.59 112.903) (end 148.590006 112.903) (width 0.25) (layer F.Cu) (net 6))
 (segment (start 148.590006 112.903) (end 148.717006 113.03) (width 0.25) (layer F.Cu) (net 6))
 (segment (start 148.3995 113.03) (end 148.717006 113.03) (width 0.25) (layer B.Cu) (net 6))
 (segment (start 147.32 111.9505) (end 148.3995 113.03) (width 0.25) (layer B.Cu) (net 6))
 (segment (start 147.32 111.533) (end 147.32 111.9505) (width 0.25) (layer B.Cu) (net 6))
 (segment (start 151.69 113.03) (end 148.717006 113.03) (width 0.25) (layer F.Cu) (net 6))
 (via (at 148.717006 113.03) (size 0.6) (drill 0.4) (layers F.Cu B.Cu) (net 6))
 (segment (start 151.69 114.3) (end 153.115 114.3) (width 0.25) (layer F.Cu) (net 5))
 (segment (start 153.115 114.3) (end 153.543 113.872) (width 0.25) (layer F.Cu) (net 5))
 (segment (start 153.543 113.872) (end 153.543 113.03) (width 0.25) (layer F.Cu) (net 5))
 (segment (start 151.13 104.14) (end 149.86 102.87) (width 0.25) (layer F.Cu) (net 5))
 (segment (start 153.543 113.03) (end 154.168001 112.404999) (width 0.25) (layer F.Cu) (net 5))
 (segment (start 151.13 106.299) (end 151.13 104.14) (width 0.25) (layer F.Cu) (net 5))
 (segment (start 154.168001 112.404999) (end 154.168001 109.337001) (width 0.25) (layer F.Cu) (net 5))
 (segment (start 154.168001 109.337001) (end 151.13 106.299) (width 0.25) (layer F.Cu) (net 5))
 (segment (start 151.429999 115.206501) (end 151.13 115.5065) (width 0.25) (layer F.Cu) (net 5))
 (segment (start 151.69 114.9465) (end 151.429999 115.206501) (width 0.25) (layer F.Cu) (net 5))
 (segment (start 151.69 114.3) (end 151.69 114.9465) (width 0.25) (layer F.Cu) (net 5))
 (segment (start 151.13 118.083) (end 151.13 115.5065) (width 0.25) (layer B.Cu) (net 5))
 (via (at 151.13 115.5065) (size 0.6) (drill 0.4) (layers F.Cu B.Cu) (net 5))
 (segment (start 149.86 105.41) (end 148.463 106.807) (width 0.25) (layer B.Cu) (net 2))
 (segment (start 148.463 106.807) (end 146.431 106.807) (width 0.25) (layer B.Cu) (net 2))
 (segment (start 146.431 106.807) (end 146.177 106.553) (width 0.25) (layer B.Cu) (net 2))
 (segment (start 146.177 106.553) (end 146.177 106.649087) (width 0.25) (layer F.Cu) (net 2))
 (segment (start 146.177 106.649087) (end 143.891 108.935087) (width 0.25) (layer F.Cu) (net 2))
 (segment (start 143.891 108.935087) (end 143.891 111.252) (width 0.25) (layer F.Cu) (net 2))
 (segment (start 143.891 111.252) (end 144.399 111.76) (width 0.25) (layer F.Cu) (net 2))
 (segment (start 144.399 111.76) (end 145.49 111.76) (width 0.25) (layer F.Cu) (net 2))
 (via (at 146.177 106.553) (size 0.6) (drill 0.4) (layers F.Cu B.Cu) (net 2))
 (segment (start 149.86 115.255) (end 149.86 115.6335) (width 0.25) (layer F.Cu) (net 2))
 (segment (start 146.365 111.76) (end 149.86 115.255) (width 0.25) (layer F.Cu) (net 2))
 (segment (start 145.49 111.76) (end 146.365 111.76) (width 0.25) (layer F.Cu) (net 2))
 (segment (start 149.86 118.083) (end 149.86 115.6335) (width 0.25) (layer B.Cu) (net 2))
 (via (at 149.86 115.6335) (size 0.6) (drill 0.4) (layers F.Cu B.Cu) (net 2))
 (segment (start 152.4 102.87) (end 151.13 104.14) (width 0.25) (layer B.Cu) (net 9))
 (segment (start 151.13 104.14) (end 151.13 106.553) (width 0.25) (layer B.Cu) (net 9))
 (segment (start 143.209 109.775) (end 143.14 109.775) (width 0.25) (layer B.Cu) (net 9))
 (segment (start 143.14 109.775) (end 142.24 109.775) (width 0.25) (layer B.Cu) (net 9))
 (segment (start 151.13 106.553) (end 150.241 107.442) (width 0.25) (layer B.Cu) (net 9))
 (segment (start 150.241 107.442) (end 145.542 107.442) (width 0.25) (layer B.Cu) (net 9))
 (segment (start 145.542 107.442) (end 143.209 109.775) (width 0.25) (layer B.Cu) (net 9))
 (segment (start 151.13 111.533) (end 151.13 110.871) (width 0.25) (layer B.Cu) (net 9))
 (segment (start 151.13 110.871) (end 151.638 110.363) (width 0.25) (layer B.Cu) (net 9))
 (segment (start 151.638 110.363) (end 153.162 110.363) (width 0.25) (layer B.Cu) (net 9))
 (segment (start 153.162 110.363) (end 153.924 111.125) (width 0.25) (layer B.Cu) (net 9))
 (segment (start 153.924 111.125) (end 155.829 111.125) (width 0.25) (layer B.Cu) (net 9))
 (segment (start 155.829 111.125) (end 156.083 110.871) (width 0.25) (layer B.Cu) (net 9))
 (segment (start 156.083 110.871) (end 156.083 104.775) (width 0.25) (layer B.Cu) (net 9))
 (segment (start 156.083 104.775) (end 154.178 102.87) (width 0.25) (layer B.Cu) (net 9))
 (segment (start 154.178 102.87) (end 152.4 102.87) (width 0.25) (layer B.Cu) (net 9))
 (segment (start 147.32 118.083) (end 147.32 117.1615) (width 0.25) (layer B.Cu) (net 9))
 (segment (start 147.32 117.1615) (end 146.685 116.5265) (width 0.25) (layer B.Cu) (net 9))
 (segment (start 146.685 116.5265) (end 146.685 110.617) (width 0.25) (layer B.Cu) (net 9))
 (segment (start 146.685 110.617) (end 146.939 110.363) (width 0.25) (layer B.Cu) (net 9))
 (segment (start 146.939 110.363) (end 149.352 110.363) (width 0.25) (layer B.Cu) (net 9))
 (segment (start 149.352 110.363) (end 149.86 110.871) (width 0.25) (layer B.Cu) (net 9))
 (segment (start 149.86 110.871) (end 149.86 111.533) (width 0.25) (layer B.Cu) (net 9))
 (segment (start 149.86 111.533) (end 151.13 111.533) (width 0.25) (layer B.Cu) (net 9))
 (segment (start 147.32 118.083) (end 146.05 118.083) (width 0.25) (layer B.Cu) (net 9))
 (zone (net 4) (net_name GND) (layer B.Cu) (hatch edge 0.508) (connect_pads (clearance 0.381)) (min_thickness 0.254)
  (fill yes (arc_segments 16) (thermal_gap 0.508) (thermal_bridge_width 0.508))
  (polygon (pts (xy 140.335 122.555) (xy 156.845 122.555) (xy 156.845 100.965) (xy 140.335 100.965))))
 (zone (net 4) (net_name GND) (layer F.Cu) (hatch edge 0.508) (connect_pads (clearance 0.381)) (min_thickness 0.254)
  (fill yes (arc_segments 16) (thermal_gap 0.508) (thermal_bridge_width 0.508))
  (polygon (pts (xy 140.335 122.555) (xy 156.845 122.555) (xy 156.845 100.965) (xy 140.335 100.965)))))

